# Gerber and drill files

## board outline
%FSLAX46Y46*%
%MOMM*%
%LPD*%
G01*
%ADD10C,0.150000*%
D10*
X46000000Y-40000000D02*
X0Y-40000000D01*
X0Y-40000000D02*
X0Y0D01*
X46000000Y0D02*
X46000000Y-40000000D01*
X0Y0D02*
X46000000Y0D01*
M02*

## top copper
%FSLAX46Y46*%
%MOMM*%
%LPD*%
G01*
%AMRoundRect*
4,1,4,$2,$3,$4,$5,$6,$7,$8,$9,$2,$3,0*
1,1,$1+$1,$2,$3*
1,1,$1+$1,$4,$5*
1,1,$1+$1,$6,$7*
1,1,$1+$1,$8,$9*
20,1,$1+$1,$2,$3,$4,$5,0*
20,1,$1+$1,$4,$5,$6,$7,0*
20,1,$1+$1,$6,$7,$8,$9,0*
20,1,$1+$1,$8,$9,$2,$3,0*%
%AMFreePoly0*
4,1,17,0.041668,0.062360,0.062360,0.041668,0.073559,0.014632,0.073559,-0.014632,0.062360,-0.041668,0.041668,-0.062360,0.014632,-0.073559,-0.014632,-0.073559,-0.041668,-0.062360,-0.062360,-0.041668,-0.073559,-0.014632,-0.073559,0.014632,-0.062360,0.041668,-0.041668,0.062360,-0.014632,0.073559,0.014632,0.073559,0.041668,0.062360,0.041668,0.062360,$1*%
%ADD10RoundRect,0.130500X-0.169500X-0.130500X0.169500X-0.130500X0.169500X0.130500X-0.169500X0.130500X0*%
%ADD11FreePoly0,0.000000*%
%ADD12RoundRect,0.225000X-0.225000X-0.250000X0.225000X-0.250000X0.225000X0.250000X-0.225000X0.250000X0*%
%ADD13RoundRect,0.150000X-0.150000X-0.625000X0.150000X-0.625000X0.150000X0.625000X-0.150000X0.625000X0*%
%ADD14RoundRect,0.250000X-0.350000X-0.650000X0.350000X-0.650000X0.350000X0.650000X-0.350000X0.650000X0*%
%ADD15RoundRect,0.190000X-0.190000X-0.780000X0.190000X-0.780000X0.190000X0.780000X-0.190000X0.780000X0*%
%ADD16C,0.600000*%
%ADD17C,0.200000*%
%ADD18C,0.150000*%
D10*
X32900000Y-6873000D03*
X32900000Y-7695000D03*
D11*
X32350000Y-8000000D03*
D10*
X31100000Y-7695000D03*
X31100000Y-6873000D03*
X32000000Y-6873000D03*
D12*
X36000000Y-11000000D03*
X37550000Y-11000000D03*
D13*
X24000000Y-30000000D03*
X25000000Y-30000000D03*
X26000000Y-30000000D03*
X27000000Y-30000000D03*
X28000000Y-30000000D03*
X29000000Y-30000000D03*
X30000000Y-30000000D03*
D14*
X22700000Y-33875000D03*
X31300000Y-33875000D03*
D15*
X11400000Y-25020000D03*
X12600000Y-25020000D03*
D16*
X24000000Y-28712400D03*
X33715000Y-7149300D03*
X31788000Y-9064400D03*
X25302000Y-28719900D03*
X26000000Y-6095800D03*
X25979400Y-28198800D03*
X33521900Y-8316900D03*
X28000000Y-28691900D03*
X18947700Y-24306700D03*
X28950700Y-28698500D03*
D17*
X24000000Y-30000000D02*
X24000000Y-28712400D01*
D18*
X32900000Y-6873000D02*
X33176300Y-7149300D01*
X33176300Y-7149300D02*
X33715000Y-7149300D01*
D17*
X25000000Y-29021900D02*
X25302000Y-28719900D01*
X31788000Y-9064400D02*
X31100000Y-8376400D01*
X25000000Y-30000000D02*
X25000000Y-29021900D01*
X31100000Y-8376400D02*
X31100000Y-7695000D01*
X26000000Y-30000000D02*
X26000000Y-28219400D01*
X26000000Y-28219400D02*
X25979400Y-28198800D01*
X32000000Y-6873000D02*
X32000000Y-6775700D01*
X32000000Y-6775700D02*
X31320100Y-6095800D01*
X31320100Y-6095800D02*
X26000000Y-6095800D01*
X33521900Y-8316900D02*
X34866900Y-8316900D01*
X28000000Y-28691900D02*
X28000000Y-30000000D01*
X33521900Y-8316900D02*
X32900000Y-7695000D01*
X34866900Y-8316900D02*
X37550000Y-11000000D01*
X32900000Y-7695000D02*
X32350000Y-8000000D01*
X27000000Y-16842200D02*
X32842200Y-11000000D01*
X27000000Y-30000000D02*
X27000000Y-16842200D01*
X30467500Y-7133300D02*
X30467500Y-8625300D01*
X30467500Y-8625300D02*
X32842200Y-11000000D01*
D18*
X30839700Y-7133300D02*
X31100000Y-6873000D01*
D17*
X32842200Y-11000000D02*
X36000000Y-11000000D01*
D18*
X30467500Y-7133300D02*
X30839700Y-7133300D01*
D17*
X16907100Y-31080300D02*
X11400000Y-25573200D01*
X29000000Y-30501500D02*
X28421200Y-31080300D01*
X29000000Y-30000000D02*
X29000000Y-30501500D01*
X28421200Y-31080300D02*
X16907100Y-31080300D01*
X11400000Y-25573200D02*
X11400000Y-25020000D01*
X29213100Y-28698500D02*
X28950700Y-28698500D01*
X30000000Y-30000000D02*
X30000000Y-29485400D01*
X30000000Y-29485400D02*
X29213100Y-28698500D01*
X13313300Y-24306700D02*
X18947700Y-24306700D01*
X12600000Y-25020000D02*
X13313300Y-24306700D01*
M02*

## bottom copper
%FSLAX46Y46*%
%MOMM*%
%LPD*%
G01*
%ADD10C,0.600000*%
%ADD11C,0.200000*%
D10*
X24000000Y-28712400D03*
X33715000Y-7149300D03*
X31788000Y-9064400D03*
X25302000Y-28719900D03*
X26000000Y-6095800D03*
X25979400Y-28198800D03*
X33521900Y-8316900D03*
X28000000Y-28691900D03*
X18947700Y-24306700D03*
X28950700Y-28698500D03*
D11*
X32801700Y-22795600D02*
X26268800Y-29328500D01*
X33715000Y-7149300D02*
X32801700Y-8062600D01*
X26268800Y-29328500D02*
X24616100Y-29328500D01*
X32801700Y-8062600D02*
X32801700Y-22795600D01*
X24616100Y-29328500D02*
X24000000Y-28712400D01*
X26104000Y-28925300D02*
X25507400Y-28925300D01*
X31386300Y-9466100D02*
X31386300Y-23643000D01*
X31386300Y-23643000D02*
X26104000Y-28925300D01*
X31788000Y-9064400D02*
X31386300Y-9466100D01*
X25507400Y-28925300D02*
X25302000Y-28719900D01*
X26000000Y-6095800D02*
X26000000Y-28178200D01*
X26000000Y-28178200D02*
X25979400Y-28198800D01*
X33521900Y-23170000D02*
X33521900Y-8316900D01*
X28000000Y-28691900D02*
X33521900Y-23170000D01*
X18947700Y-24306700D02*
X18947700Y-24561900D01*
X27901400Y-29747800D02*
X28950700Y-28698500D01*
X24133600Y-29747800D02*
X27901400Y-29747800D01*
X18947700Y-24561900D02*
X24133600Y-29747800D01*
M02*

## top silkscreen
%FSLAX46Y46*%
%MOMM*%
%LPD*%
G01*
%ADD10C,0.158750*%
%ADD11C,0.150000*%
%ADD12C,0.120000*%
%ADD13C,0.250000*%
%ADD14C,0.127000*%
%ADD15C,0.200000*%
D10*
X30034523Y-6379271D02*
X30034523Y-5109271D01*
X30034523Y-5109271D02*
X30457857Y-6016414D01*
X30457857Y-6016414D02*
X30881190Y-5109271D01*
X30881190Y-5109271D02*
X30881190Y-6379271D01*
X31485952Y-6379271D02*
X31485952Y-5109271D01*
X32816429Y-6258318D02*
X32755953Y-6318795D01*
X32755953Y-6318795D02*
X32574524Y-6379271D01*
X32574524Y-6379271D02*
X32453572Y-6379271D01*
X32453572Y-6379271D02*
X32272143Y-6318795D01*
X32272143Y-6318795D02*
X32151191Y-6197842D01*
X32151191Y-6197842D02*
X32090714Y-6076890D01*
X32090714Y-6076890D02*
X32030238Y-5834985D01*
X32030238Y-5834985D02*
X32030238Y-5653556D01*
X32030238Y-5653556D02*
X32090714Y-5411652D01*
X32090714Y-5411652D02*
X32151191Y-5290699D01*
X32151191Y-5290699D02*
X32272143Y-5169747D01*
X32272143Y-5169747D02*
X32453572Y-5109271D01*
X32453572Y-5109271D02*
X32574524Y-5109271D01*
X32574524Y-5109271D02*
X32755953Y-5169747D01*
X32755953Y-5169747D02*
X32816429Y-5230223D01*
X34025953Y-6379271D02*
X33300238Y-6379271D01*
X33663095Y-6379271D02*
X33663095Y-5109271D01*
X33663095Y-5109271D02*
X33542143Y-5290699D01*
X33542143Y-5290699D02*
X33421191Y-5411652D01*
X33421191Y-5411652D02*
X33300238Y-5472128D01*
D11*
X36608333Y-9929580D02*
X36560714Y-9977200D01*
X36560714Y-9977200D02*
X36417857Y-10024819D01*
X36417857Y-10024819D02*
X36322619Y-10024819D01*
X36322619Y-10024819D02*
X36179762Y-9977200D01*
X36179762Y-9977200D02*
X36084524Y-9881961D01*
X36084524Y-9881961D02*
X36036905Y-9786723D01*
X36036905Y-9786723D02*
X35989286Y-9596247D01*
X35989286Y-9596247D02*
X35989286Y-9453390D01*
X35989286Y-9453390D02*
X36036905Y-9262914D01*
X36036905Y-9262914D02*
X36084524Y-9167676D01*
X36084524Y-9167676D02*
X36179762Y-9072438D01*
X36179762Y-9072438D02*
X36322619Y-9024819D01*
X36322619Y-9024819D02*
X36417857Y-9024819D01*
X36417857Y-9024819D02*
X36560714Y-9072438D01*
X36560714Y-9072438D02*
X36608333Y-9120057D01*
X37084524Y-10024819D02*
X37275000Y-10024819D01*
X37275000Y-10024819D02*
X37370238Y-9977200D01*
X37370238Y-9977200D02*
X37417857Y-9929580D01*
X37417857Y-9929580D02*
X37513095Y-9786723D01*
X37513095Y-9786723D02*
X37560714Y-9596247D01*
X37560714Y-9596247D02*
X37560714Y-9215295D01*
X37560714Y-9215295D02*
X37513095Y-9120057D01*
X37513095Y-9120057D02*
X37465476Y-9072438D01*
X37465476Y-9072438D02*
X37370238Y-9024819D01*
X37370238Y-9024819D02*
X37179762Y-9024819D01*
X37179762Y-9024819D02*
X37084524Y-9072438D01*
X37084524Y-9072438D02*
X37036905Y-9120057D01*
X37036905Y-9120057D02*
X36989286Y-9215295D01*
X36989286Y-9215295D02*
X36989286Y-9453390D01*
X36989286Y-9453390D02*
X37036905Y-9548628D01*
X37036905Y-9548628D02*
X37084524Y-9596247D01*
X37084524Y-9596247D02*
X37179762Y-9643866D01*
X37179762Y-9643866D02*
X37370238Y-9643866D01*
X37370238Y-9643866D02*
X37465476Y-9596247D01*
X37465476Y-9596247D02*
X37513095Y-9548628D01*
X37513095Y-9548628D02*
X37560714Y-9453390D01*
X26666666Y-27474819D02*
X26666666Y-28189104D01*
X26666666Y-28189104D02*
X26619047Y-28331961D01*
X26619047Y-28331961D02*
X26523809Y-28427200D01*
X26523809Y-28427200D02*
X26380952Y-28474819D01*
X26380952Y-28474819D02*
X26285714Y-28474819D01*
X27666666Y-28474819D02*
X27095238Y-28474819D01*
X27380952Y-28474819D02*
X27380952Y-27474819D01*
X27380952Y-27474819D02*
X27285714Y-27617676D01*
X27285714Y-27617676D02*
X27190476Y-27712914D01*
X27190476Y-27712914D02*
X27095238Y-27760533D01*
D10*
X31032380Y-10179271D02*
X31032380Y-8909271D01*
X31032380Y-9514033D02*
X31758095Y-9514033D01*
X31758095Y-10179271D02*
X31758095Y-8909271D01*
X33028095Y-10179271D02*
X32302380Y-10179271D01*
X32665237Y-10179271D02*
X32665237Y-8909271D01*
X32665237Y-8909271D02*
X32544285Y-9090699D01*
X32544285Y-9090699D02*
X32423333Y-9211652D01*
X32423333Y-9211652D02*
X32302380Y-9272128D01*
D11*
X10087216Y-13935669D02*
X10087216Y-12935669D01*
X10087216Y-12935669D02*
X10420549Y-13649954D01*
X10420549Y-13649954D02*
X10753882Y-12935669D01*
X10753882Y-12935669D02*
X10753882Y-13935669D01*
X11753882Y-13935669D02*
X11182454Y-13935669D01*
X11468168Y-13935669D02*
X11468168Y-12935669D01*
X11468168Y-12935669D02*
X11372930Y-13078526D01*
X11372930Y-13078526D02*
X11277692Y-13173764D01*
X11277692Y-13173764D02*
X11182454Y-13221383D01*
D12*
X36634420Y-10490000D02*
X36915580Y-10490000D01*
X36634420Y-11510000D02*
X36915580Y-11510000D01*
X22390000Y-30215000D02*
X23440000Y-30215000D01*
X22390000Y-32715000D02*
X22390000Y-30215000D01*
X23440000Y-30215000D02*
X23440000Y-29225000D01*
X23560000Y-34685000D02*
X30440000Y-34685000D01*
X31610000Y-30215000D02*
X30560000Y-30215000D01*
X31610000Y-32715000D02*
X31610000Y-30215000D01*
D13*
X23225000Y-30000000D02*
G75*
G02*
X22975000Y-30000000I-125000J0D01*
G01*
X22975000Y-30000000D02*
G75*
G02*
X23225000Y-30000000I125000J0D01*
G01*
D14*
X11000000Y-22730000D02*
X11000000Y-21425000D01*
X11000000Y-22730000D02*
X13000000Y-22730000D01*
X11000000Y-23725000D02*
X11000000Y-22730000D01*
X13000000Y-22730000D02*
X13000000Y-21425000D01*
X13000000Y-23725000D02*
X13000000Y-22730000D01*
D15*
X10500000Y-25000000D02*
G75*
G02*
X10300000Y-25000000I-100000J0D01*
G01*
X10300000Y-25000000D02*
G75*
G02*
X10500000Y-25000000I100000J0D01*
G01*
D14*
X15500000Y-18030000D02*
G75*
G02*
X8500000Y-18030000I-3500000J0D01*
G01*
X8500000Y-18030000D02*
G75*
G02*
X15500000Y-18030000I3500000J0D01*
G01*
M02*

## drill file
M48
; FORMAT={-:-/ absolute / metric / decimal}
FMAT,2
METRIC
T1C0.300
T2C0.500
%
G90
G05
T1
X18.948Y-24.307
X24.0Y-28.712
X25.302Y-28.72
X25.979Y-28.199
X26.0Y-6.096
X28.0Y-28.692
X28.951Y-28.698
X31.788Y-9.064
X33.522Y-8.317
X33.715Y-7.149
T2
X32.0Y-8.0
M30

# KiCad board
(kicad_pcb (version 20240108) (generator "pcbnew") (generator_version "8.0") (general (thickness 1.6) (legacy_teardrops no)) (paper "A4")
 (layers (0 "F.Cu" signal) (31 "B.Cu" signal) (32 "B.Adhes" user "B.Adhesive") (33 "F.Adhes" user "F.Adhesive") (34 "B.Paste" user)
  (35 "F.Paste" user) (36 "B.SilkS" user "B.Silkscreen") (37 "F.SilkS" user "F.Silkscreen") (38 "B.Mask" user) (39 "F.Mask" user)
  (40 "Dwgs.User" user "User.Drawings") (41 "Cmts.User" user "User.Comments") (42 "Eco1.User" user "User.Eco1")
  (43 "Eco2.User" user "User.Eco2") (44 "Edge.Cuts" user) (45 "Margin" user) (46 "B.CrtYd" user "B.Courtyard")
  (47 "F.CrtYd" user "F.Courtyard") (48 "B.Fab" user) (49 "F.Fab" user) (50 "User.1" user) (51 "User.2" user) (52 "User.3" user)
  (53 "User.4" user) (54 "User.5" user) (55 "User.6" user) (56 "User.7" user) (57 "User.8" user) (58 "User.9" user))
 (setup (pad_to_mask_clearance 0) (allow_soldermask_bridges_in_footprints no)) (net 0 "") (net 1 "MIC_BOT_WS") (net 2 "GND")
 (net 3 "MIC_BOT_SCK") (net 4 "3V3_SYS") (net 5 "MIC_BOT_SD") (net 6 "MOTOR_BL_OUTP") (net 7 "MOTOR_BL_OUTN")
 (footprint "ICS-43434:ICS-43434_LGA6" (layer "F.Cu") (at 32 8)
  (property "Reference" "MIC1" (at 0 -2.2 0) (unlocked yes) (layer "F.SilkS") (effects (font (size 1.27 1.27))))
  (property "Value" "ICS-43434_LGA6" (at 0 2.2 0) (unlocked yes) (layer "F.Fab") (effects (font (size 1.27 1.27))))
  (pad "1" smd roundrect (at 0.9 -1.127) (size 0.6 0.522) (layers "F.Cu" "F.Paste" "F.Mask") (roundrect_rratio 0.25) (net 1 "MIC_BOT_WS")
   (thermal_bridge_angle 45))
  (pad "2" smd roundrect (at 0.9 -0.305) (size 0.6 0.522) (layers "F.Cu" "F.Paste" "F.Mask") (roundrect_rratio 0.25) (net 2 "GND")
   (thermal_bridge_angle 45))
  (pad "3" smd custom (at 0.35 0) (size 0.15 0.15) (layers "F.Cu" "F.Mask") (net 2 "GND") (options (clearance outline) (anchor circle))
   (primitives))
  (pad "4" smd roundrect (at -0.9 -0.305) (size 0.6 0.522) (layers "F.Cu" "F.Paste" "F.Mask") (roundrect_rratio 0.25) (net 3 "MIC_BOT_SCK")
   (thermal_bridge_angle 45))
  (pad "5" smd roundrect (at -0.9 -1.127) (size 0.6 0.522) (layers "F.Cu" "F.Paste" "F.Mask") (roundrect_rratio 0.25) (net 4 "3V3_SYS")
   (thermal_bridge_angle 45))
  (pad "6" smd roundrect (at 0 -1.127) (size 0.6 0.522) (layers "F.Cu" "F.Paste" "F.Mask") (roundrect_rratio 0.25) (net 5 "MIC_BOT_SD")
   (thermal_bridge_angle 45)))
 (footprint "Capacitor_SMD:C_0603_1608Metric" (layer "F.Cu") (at 36.775 11)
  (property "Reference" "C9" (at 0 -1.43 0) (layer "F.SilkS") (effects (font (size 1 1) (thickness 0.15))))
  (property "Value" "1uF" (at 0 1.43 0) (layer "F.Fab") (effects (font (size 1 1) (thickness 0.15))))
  (fp_line (start -0.14058 -0.51) (end 0.14058 -0.51) (stroke (width 0.12) (type solid)) (layer "F.SilkS"))
  (fp_line (start -0.14058 0.51) (end 0.14058 0.51) (stroke (width 0.12) (type solid)) (layer "F.SilkS"))
  (pad "1" smd roundrect (at -0.775 0) (size 0.9 0.95) (layers "F.Cu" "F.Paste" "F.Mask") (roundrect_rratio 0.25) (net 4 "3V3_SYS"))
  (pad "2" smd roundrect (at 0.775 0) (size 0.9 0.95) (layers "F.Cu" "F.Paste" "F.Mask") (roundrect_rratio 0.25) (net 2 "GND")))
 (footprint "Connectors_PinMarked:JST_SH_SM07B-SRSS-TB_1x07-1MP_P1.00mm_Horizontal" (layer "F.Cu") (at 27 32)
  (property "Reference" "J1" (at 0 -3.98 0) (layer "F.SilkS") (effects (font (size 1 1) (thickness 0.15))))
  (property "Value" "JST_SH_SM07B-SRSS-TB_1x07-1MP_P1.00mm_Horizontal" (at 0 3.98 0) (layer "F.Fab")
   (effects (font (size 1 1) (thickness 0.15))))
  (fp_line (start -4.61 -1.785) (end -3.56 -1.785) (stroke (width 0.12) (type solid)) (layer "F.SilkS"))
  (fp_line (start -4.61 0.715) (end -4.61 -1.785) (stroke (width 0.12) (type solid)) (layer "F.SilkS"))
  (fp_line (start -3.56 -1.785) (end -3.56 -2.775) (stroke (width 0.12) (type solid)) (layer "F.SilkS"))
  (fp_line (start -3.44 2.685) (end 3.44 2.685) (stroke (width 0.12) (type solid)) (layer "F.SilkS"))
  (fp_line (start 4.61 -1.785) (end 3.56 -1.785) (stroke (width 0.12) (type solid)) (layer "F.SilkS"))
  (fp_line (start 4.61 0.715) (end 4.61 -1.785) (stroke (width 0.12) (type solid)) (layer "F.SilkS"))
  (fp_circle (center -3.9 -2) (end -3.7 -2) (stroke (width 0.1) (type solid)) (fill solid) (layer "F.SilkS"))
  (pad "1" smd roundrect (at -3 -2) (size 0.6 1.55) (layers "F.Cu" "F.Paste" "F.Mask") (roundrect_rratio 0.25) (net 1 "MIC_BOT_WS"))
  (pad "2" smd roundrect (at -2 -2) (size 0.6 1.55) (layers "F.Cu" "F.Paste" "F.Mask") (roundrect_rratio 0.25) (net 3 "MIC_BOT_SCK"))
  (pad "3" smd roundrect (at -1 -2) (size 0.6 1.55) (layers "F.Cu" "F.Paste" "F.Mask") (roundrect_rratio 0.25) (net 5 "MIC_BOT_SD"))
  (pad "4" smd roundrect (at 0 -2) (size 0.6 1.55) (layers "F.Cu" "F.Paste" "F.Mask") (roundrect_rratio 0.25) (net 4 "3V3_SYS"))
  (pad "5" smd roundrect (at 1 -2) (size 0.6 1.55) (layers "F.Cu" "F.Paste" "F.Mask") (roundrect_rratio 0.25) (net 2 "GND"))
  (pad "6" smd roundrect (at 2 -2) (size 0.6 1.55) (layers "F.Cu" "F.Paste" "F.Mask") (roundrect_rratio 0.25) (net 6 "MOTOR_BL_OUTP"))
  (pad "7" smd roundrect (at 3 -2) (size 0.6 1.55) (layers "F.Cu" "F.Paste" "F.Mask") (roundrect_rratio 0.25) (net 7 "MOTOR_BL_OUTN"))
  (pad "MP" smd roundrect (at -4.3 1.875) (size 1.2 1.8) (layers "F.Cu" "F.Paste" "F.Mask") (roundrect_rratio 0.208333))
  (pad "MP" smd roundrect (at 4.3 1.875) (size 1.2 1.8) (layers "F.Cu" "F.Paste" "F.Mask") (roundrect_rratio 0.208333)))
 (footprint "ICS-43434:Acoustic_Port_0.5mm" (layer "F.Cu") (at 32 8)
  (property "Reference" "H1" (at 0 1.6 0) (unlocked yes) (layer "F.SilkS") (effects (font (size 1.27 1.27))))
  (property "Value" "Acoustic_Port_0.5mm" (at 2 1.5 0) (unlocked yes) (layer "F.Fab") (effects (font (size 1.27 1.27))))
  (pad "" np_thru_hole circle (at 0 0) (size 0.5 0.5) (drill 0.5) (layers "*.Cu" "*.Mask")))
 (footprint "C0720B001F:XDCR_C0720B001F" (layer "F.Cu") (at 12 20)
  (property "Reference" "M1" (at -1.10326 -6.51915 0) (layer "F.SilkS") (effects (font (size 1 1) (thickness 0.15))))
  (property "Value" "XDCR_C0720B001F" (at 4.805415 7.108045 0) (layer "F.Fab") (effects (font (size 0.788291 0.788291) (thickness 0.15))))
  (fp_line (start -1 2.73) (end -1 1.425) (stroke (width 0.127) (type solid)) (layer "F.SilkS"))
  (fp_line (start -1 2.73) (end 1 2.73) (stroke (width 0.127) (type solid)) (layer "F.SilkS"))
  (fp_line (start -1 3.725) (end -1 2.73) (stroke (width 0.127) (type solid)) (layer "F.SilkS"))
  (fp_line (start 1 2.73) (end 1 1.425) (stroke (width 0.127) (type solid)) (layer "F.SilkS"))
  (fp_line (start 1 3.725) (end 1 2.73) (stroke (width 0.127) (type solid)) (layer "F.SilkS"))
  (fp_circle (center -1.6 5) (end -1.5 5) (stroke (width 0.2) (type solid)) (fill none) (layer "F.SilkS"))
  (fp_circle (center 0 -1.97) (end 3.5 -1.97) (stroke (width 0.127) (type solid)) (fill none) (layer "F.SilkS"))
  (pad "1" smd roundrect (at -0.6 5.02) (size 0.76 1.94) (layers "F.Cu" "F.Paste" "F.Mask") (roundrect_rratio 0.25) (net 6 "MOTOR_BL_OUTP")
   (solder_mask_margin 0.102))
  (pad "2" smd roundrect (at 0.6 5.02) (size 0.76 1.94) (layers "F.Cu" "F.Paste" "F.Mask") (roundrect_rratio 0.25) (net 7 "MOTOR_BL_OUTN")
   (solder_mask_margin 0.102)))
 (gr_line (start 46 40) (end 0 40) (stroke (width 0.15) (type default)) (layer "Edge.Cuts"))
 (gr_line (start 0 40) (end 0 0) (stroke (width 0.15) (type default)) (layer "Edge.Cuts"))
 (gr_line (start 46 0) (end 46 40) (stroke (width 0.15) (type default)) (layer "Edge.Cuts"))
 (gr_line (start 0 0) (end 46 0) (stroke (width 0.15) (type default)) (layer "Edge.Cuts"))
 (segment (start 24 30) (end 24 28.7124) (width 0.2) (layer "F.Cu") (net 1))
 (segment (start 32.9 6.873) (end 33.1763 7.1493) (width 0.15) (layer "F.Cu") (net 1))
 (segment (start 33.1763 7.1493) (end 33.715 7.1493) (width 0.15) (layer "F.Cu") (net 1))
 (via (at 24 28.7124) (size 0.6) (drill 0.3) (layers "F.Cu" "B.Cu") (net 1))
 (via (at 33.715 7.1493) (size 0.6) (drill 0.3) (layers "F.Cu" "B.Cu") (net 1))
 (segment (start 32.8017 22.7956) (end 26.2688 29.3285) (width 0.2) (layer "B.Cu") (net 1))
 (segment (start 33.715 7.1493) (end 32.8017 8.0626) (width 0.2) (layer "B.Cu") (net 1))
 (segment (start 26.2688 29.3285) (end 24.6161 29.3285) (width 0.2) (layer "B.Cu") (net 1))
 (segment (start 32.8017 8.0626) (end 32.8017 22.7956) (width 0.2) (layer "B.Cu") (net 1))
 (segment (start 24.6161 29.3285) (end 24 28.7124) (width 0.2) (layer "B.Cu") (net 1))
 (segment (start 25 29.0219) (end 25.302 28.7199) (width 0.2) (layer "F.Cu") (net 3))
 (segment (start 31.788 9.0644) (end 31.1 8.3764) (width 0.2) (layer "F.Cu") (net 3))
 (segment (start 25 30) (end 25 29.0219) (width 0.2) (layer "F.Cu") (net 3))
 (segment (start 31.1 8.3764) (end 31.1 7.695) (width 0.2) (layer "F.Cu") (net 3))
 (via (at 31.788 9.0644) (size 0.6) (drill 0.3) (layers "F.Cu" "B.Cu") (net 3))
 (via (at 25.302 28.7199) (size 0.6) (drill 0.3) (layers "F.Cu" "B.Cu") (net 3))
 (segment (start 26.104 28.9253) (end 25.5074 28.9253) (width 0.2) (layer "B.Cu") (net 3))
 (segment (start 31.3863 9.4661) (end 31.3863 23.643) (width 0.2) (layer "B.Cu") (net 3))
 (segment (start 31.3863 23.643) (end 26.104 28.9253) (width 0.2) (layer "B.Cu") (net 3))
 (segment (start 31.788 9.0644) (end 31.3863 9.4661) (width 0.2) (layer "B.Cu") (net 3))
 (segment (start 25.5074 28.9253) (end 25.302 28.7199) (width 0.2) (layer "B.Cu") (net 3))
 (segment (start 26 30) (end 26 28.2194) (width 0.2) (layer "F.Cu") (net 5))
 (segment (start 26 28.2194) (end 25.9794 28.1988) (width 0.2) (layer "F.Cu") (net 5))
 (segment (start 32 6.873) (end 32 6.7757) (width 0.2) (layer "F.Cu") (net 5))
 (segment (start 32 6.7757) (end 31.3201 6.0958) (width 0.2) (layer "F.Cu") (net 5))
 (segment (start 31.3201 6.0958) (end 26 6.0958) (width 0.2) (layer "F.Cu") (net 5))
 (via (at 26 6.0958) (size 0.6) (drill 0.3) (layers "F.Cu" "B.Cu") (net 5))
 (via (at 25.9794 28.1988) (size 0.6) (drill 0.3) (layers "F.Cu" "B.Cu") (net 5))
 (segment (start 26 6.0958) (end 26 28.1782) (width 0.2) (layer "B.Cu") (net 5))
 (segment (start 26 28.1782) (end 25.9794 28.1988) (width 0.2) (layer "B.Cu") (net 5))
 (segment (start 33.5219 8.3169) (end 34.8669 8.3169) (width 0.2) (layer "F.Cu") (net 2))
 (segment (start 28 28.6919) (end 28 30) (width 0.2) (layer "F.Cu") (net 2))
 (segment (start 33.5219 8.3169) (end 32.9 7.695) (width 0.2) (layer "F.Cu") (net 2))
 (segment (start 34.8669 8.3169) (end 37.55 11) (width 0.2) (layer "F.Cu") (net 2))
 (segment (start 32.9 7.695) (end 32.35 8) (width 0.2) (layer "F.Cu") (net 2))
 (via (at 33.5219 8.3169) (size 0.6) (drill 0.3) (layers "F.Cu" "B.Cu") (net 2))
 (via (at 28 28.6919) (size 0.6) (drill 0.3) (layers "F.Cu" "B.Cu") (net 2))
 (segment (start 33.5219 23.17) (end 33.5219 8.3169) (width 0.2) (layer "B.Cu") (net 2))
 (segment (start 28 28.6919) (end 33.5219 23.17) (width 0.2) (layer "B.Cu") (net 2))
 (segment (start 27 16.8422) (end 32.8422 11) (width 0.2) (layer "F.Cu") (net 4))
 (segment (start 27 30) (end 27 16.8422) (width 0.2) (layer "F.Cu") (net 4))
 (segment (start 30.4675 7.1333) (end 30.4675 8.6253) (width 0.2) (layer "F.Cu") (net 4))
 (segment (start 30.4675 8.6253) (end 32.8422 11) (width 0.2) (layer "F.Cu") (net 4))
 (segment (start 30.8397 7.1333) (end 31.1 6.873) (width 0.15) (layer "F.Cu") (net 4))
 (segment (start 32.8422 11) (end 36 11) (width 0.2) (layer "F.Cu") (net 4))
 (segment (start 30.4675 7.1333) (end 30.8397 7.1333) (width 0.15) (layer "F.Cu") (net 4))
 (segment (start 16.9071 31.0803) (end 11.4 25.5732) (width 0.2) (layer "F.Cu") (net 6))
 (segment (start 29 30.5015) (end 28.4212 31.0803) (width 0.2) (layer "F.Cu") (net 6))
 (segment (start 29 30) (end 29 30.5015) (width 0.2) (layer "F.Cu") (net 6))
 (segment (start 28.4212 31.0803) (end 16.9071 31.0803) (width 0.2) (layer "F.Cu") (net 6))
 (segment (start 11.4 25.5732) (end 11.4 25.02) (width 0.2) (layer "F.Cu") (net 6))
 (segment (start 29.2131 28.6985) (end 28.9507 28.6985) (width 0.2) (layer "F.Cu") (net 7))
 (segment (start 30 30) (end 30 29.4854) (width 0.2) (layer "F.Cu") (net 7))
 (segment (start 30 29.4854) (end 29.2131 28.6985) (width 0.2) (layer "F.Cu") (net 7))
 (segment (start 13.3133 24.3067) (end 18.9477 24.3067) (width 0.2) (layer "F.Cu") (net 7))
 (segment (start 12.6 25.02) (end 13.3133 24.3067) (width 0.2) (layer "F.Cu") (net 7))
 (via (at 18.9477 24.3067) (size 0.6) (drill 0.3) (layers "F.Cu" "B.Cu") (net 7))
 (via (at 28.9507 28.6985) (size 0.6) (drill 0.3) (layers "F.Cu" "B.Cu") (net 7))
 (segment (start 18.9477 24.3067) (end 18.9477 24.5619) (width 0.2) (layer "B.Cu") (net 7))
 (segment (start 27.9014 29.7478) (end 28.9507 28.6985) (width 0.2) (layer "B.Cu") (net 7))
 (segment (start 24.1336 29.7478) (end 27.9014 29.7478) (width 0.2) (layer "B.Cu") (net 7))
 (segment (start 18.9477 24.5619) (end 24.1336 29.7478) (width 0.2) (layer "B.Cu") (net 7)))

